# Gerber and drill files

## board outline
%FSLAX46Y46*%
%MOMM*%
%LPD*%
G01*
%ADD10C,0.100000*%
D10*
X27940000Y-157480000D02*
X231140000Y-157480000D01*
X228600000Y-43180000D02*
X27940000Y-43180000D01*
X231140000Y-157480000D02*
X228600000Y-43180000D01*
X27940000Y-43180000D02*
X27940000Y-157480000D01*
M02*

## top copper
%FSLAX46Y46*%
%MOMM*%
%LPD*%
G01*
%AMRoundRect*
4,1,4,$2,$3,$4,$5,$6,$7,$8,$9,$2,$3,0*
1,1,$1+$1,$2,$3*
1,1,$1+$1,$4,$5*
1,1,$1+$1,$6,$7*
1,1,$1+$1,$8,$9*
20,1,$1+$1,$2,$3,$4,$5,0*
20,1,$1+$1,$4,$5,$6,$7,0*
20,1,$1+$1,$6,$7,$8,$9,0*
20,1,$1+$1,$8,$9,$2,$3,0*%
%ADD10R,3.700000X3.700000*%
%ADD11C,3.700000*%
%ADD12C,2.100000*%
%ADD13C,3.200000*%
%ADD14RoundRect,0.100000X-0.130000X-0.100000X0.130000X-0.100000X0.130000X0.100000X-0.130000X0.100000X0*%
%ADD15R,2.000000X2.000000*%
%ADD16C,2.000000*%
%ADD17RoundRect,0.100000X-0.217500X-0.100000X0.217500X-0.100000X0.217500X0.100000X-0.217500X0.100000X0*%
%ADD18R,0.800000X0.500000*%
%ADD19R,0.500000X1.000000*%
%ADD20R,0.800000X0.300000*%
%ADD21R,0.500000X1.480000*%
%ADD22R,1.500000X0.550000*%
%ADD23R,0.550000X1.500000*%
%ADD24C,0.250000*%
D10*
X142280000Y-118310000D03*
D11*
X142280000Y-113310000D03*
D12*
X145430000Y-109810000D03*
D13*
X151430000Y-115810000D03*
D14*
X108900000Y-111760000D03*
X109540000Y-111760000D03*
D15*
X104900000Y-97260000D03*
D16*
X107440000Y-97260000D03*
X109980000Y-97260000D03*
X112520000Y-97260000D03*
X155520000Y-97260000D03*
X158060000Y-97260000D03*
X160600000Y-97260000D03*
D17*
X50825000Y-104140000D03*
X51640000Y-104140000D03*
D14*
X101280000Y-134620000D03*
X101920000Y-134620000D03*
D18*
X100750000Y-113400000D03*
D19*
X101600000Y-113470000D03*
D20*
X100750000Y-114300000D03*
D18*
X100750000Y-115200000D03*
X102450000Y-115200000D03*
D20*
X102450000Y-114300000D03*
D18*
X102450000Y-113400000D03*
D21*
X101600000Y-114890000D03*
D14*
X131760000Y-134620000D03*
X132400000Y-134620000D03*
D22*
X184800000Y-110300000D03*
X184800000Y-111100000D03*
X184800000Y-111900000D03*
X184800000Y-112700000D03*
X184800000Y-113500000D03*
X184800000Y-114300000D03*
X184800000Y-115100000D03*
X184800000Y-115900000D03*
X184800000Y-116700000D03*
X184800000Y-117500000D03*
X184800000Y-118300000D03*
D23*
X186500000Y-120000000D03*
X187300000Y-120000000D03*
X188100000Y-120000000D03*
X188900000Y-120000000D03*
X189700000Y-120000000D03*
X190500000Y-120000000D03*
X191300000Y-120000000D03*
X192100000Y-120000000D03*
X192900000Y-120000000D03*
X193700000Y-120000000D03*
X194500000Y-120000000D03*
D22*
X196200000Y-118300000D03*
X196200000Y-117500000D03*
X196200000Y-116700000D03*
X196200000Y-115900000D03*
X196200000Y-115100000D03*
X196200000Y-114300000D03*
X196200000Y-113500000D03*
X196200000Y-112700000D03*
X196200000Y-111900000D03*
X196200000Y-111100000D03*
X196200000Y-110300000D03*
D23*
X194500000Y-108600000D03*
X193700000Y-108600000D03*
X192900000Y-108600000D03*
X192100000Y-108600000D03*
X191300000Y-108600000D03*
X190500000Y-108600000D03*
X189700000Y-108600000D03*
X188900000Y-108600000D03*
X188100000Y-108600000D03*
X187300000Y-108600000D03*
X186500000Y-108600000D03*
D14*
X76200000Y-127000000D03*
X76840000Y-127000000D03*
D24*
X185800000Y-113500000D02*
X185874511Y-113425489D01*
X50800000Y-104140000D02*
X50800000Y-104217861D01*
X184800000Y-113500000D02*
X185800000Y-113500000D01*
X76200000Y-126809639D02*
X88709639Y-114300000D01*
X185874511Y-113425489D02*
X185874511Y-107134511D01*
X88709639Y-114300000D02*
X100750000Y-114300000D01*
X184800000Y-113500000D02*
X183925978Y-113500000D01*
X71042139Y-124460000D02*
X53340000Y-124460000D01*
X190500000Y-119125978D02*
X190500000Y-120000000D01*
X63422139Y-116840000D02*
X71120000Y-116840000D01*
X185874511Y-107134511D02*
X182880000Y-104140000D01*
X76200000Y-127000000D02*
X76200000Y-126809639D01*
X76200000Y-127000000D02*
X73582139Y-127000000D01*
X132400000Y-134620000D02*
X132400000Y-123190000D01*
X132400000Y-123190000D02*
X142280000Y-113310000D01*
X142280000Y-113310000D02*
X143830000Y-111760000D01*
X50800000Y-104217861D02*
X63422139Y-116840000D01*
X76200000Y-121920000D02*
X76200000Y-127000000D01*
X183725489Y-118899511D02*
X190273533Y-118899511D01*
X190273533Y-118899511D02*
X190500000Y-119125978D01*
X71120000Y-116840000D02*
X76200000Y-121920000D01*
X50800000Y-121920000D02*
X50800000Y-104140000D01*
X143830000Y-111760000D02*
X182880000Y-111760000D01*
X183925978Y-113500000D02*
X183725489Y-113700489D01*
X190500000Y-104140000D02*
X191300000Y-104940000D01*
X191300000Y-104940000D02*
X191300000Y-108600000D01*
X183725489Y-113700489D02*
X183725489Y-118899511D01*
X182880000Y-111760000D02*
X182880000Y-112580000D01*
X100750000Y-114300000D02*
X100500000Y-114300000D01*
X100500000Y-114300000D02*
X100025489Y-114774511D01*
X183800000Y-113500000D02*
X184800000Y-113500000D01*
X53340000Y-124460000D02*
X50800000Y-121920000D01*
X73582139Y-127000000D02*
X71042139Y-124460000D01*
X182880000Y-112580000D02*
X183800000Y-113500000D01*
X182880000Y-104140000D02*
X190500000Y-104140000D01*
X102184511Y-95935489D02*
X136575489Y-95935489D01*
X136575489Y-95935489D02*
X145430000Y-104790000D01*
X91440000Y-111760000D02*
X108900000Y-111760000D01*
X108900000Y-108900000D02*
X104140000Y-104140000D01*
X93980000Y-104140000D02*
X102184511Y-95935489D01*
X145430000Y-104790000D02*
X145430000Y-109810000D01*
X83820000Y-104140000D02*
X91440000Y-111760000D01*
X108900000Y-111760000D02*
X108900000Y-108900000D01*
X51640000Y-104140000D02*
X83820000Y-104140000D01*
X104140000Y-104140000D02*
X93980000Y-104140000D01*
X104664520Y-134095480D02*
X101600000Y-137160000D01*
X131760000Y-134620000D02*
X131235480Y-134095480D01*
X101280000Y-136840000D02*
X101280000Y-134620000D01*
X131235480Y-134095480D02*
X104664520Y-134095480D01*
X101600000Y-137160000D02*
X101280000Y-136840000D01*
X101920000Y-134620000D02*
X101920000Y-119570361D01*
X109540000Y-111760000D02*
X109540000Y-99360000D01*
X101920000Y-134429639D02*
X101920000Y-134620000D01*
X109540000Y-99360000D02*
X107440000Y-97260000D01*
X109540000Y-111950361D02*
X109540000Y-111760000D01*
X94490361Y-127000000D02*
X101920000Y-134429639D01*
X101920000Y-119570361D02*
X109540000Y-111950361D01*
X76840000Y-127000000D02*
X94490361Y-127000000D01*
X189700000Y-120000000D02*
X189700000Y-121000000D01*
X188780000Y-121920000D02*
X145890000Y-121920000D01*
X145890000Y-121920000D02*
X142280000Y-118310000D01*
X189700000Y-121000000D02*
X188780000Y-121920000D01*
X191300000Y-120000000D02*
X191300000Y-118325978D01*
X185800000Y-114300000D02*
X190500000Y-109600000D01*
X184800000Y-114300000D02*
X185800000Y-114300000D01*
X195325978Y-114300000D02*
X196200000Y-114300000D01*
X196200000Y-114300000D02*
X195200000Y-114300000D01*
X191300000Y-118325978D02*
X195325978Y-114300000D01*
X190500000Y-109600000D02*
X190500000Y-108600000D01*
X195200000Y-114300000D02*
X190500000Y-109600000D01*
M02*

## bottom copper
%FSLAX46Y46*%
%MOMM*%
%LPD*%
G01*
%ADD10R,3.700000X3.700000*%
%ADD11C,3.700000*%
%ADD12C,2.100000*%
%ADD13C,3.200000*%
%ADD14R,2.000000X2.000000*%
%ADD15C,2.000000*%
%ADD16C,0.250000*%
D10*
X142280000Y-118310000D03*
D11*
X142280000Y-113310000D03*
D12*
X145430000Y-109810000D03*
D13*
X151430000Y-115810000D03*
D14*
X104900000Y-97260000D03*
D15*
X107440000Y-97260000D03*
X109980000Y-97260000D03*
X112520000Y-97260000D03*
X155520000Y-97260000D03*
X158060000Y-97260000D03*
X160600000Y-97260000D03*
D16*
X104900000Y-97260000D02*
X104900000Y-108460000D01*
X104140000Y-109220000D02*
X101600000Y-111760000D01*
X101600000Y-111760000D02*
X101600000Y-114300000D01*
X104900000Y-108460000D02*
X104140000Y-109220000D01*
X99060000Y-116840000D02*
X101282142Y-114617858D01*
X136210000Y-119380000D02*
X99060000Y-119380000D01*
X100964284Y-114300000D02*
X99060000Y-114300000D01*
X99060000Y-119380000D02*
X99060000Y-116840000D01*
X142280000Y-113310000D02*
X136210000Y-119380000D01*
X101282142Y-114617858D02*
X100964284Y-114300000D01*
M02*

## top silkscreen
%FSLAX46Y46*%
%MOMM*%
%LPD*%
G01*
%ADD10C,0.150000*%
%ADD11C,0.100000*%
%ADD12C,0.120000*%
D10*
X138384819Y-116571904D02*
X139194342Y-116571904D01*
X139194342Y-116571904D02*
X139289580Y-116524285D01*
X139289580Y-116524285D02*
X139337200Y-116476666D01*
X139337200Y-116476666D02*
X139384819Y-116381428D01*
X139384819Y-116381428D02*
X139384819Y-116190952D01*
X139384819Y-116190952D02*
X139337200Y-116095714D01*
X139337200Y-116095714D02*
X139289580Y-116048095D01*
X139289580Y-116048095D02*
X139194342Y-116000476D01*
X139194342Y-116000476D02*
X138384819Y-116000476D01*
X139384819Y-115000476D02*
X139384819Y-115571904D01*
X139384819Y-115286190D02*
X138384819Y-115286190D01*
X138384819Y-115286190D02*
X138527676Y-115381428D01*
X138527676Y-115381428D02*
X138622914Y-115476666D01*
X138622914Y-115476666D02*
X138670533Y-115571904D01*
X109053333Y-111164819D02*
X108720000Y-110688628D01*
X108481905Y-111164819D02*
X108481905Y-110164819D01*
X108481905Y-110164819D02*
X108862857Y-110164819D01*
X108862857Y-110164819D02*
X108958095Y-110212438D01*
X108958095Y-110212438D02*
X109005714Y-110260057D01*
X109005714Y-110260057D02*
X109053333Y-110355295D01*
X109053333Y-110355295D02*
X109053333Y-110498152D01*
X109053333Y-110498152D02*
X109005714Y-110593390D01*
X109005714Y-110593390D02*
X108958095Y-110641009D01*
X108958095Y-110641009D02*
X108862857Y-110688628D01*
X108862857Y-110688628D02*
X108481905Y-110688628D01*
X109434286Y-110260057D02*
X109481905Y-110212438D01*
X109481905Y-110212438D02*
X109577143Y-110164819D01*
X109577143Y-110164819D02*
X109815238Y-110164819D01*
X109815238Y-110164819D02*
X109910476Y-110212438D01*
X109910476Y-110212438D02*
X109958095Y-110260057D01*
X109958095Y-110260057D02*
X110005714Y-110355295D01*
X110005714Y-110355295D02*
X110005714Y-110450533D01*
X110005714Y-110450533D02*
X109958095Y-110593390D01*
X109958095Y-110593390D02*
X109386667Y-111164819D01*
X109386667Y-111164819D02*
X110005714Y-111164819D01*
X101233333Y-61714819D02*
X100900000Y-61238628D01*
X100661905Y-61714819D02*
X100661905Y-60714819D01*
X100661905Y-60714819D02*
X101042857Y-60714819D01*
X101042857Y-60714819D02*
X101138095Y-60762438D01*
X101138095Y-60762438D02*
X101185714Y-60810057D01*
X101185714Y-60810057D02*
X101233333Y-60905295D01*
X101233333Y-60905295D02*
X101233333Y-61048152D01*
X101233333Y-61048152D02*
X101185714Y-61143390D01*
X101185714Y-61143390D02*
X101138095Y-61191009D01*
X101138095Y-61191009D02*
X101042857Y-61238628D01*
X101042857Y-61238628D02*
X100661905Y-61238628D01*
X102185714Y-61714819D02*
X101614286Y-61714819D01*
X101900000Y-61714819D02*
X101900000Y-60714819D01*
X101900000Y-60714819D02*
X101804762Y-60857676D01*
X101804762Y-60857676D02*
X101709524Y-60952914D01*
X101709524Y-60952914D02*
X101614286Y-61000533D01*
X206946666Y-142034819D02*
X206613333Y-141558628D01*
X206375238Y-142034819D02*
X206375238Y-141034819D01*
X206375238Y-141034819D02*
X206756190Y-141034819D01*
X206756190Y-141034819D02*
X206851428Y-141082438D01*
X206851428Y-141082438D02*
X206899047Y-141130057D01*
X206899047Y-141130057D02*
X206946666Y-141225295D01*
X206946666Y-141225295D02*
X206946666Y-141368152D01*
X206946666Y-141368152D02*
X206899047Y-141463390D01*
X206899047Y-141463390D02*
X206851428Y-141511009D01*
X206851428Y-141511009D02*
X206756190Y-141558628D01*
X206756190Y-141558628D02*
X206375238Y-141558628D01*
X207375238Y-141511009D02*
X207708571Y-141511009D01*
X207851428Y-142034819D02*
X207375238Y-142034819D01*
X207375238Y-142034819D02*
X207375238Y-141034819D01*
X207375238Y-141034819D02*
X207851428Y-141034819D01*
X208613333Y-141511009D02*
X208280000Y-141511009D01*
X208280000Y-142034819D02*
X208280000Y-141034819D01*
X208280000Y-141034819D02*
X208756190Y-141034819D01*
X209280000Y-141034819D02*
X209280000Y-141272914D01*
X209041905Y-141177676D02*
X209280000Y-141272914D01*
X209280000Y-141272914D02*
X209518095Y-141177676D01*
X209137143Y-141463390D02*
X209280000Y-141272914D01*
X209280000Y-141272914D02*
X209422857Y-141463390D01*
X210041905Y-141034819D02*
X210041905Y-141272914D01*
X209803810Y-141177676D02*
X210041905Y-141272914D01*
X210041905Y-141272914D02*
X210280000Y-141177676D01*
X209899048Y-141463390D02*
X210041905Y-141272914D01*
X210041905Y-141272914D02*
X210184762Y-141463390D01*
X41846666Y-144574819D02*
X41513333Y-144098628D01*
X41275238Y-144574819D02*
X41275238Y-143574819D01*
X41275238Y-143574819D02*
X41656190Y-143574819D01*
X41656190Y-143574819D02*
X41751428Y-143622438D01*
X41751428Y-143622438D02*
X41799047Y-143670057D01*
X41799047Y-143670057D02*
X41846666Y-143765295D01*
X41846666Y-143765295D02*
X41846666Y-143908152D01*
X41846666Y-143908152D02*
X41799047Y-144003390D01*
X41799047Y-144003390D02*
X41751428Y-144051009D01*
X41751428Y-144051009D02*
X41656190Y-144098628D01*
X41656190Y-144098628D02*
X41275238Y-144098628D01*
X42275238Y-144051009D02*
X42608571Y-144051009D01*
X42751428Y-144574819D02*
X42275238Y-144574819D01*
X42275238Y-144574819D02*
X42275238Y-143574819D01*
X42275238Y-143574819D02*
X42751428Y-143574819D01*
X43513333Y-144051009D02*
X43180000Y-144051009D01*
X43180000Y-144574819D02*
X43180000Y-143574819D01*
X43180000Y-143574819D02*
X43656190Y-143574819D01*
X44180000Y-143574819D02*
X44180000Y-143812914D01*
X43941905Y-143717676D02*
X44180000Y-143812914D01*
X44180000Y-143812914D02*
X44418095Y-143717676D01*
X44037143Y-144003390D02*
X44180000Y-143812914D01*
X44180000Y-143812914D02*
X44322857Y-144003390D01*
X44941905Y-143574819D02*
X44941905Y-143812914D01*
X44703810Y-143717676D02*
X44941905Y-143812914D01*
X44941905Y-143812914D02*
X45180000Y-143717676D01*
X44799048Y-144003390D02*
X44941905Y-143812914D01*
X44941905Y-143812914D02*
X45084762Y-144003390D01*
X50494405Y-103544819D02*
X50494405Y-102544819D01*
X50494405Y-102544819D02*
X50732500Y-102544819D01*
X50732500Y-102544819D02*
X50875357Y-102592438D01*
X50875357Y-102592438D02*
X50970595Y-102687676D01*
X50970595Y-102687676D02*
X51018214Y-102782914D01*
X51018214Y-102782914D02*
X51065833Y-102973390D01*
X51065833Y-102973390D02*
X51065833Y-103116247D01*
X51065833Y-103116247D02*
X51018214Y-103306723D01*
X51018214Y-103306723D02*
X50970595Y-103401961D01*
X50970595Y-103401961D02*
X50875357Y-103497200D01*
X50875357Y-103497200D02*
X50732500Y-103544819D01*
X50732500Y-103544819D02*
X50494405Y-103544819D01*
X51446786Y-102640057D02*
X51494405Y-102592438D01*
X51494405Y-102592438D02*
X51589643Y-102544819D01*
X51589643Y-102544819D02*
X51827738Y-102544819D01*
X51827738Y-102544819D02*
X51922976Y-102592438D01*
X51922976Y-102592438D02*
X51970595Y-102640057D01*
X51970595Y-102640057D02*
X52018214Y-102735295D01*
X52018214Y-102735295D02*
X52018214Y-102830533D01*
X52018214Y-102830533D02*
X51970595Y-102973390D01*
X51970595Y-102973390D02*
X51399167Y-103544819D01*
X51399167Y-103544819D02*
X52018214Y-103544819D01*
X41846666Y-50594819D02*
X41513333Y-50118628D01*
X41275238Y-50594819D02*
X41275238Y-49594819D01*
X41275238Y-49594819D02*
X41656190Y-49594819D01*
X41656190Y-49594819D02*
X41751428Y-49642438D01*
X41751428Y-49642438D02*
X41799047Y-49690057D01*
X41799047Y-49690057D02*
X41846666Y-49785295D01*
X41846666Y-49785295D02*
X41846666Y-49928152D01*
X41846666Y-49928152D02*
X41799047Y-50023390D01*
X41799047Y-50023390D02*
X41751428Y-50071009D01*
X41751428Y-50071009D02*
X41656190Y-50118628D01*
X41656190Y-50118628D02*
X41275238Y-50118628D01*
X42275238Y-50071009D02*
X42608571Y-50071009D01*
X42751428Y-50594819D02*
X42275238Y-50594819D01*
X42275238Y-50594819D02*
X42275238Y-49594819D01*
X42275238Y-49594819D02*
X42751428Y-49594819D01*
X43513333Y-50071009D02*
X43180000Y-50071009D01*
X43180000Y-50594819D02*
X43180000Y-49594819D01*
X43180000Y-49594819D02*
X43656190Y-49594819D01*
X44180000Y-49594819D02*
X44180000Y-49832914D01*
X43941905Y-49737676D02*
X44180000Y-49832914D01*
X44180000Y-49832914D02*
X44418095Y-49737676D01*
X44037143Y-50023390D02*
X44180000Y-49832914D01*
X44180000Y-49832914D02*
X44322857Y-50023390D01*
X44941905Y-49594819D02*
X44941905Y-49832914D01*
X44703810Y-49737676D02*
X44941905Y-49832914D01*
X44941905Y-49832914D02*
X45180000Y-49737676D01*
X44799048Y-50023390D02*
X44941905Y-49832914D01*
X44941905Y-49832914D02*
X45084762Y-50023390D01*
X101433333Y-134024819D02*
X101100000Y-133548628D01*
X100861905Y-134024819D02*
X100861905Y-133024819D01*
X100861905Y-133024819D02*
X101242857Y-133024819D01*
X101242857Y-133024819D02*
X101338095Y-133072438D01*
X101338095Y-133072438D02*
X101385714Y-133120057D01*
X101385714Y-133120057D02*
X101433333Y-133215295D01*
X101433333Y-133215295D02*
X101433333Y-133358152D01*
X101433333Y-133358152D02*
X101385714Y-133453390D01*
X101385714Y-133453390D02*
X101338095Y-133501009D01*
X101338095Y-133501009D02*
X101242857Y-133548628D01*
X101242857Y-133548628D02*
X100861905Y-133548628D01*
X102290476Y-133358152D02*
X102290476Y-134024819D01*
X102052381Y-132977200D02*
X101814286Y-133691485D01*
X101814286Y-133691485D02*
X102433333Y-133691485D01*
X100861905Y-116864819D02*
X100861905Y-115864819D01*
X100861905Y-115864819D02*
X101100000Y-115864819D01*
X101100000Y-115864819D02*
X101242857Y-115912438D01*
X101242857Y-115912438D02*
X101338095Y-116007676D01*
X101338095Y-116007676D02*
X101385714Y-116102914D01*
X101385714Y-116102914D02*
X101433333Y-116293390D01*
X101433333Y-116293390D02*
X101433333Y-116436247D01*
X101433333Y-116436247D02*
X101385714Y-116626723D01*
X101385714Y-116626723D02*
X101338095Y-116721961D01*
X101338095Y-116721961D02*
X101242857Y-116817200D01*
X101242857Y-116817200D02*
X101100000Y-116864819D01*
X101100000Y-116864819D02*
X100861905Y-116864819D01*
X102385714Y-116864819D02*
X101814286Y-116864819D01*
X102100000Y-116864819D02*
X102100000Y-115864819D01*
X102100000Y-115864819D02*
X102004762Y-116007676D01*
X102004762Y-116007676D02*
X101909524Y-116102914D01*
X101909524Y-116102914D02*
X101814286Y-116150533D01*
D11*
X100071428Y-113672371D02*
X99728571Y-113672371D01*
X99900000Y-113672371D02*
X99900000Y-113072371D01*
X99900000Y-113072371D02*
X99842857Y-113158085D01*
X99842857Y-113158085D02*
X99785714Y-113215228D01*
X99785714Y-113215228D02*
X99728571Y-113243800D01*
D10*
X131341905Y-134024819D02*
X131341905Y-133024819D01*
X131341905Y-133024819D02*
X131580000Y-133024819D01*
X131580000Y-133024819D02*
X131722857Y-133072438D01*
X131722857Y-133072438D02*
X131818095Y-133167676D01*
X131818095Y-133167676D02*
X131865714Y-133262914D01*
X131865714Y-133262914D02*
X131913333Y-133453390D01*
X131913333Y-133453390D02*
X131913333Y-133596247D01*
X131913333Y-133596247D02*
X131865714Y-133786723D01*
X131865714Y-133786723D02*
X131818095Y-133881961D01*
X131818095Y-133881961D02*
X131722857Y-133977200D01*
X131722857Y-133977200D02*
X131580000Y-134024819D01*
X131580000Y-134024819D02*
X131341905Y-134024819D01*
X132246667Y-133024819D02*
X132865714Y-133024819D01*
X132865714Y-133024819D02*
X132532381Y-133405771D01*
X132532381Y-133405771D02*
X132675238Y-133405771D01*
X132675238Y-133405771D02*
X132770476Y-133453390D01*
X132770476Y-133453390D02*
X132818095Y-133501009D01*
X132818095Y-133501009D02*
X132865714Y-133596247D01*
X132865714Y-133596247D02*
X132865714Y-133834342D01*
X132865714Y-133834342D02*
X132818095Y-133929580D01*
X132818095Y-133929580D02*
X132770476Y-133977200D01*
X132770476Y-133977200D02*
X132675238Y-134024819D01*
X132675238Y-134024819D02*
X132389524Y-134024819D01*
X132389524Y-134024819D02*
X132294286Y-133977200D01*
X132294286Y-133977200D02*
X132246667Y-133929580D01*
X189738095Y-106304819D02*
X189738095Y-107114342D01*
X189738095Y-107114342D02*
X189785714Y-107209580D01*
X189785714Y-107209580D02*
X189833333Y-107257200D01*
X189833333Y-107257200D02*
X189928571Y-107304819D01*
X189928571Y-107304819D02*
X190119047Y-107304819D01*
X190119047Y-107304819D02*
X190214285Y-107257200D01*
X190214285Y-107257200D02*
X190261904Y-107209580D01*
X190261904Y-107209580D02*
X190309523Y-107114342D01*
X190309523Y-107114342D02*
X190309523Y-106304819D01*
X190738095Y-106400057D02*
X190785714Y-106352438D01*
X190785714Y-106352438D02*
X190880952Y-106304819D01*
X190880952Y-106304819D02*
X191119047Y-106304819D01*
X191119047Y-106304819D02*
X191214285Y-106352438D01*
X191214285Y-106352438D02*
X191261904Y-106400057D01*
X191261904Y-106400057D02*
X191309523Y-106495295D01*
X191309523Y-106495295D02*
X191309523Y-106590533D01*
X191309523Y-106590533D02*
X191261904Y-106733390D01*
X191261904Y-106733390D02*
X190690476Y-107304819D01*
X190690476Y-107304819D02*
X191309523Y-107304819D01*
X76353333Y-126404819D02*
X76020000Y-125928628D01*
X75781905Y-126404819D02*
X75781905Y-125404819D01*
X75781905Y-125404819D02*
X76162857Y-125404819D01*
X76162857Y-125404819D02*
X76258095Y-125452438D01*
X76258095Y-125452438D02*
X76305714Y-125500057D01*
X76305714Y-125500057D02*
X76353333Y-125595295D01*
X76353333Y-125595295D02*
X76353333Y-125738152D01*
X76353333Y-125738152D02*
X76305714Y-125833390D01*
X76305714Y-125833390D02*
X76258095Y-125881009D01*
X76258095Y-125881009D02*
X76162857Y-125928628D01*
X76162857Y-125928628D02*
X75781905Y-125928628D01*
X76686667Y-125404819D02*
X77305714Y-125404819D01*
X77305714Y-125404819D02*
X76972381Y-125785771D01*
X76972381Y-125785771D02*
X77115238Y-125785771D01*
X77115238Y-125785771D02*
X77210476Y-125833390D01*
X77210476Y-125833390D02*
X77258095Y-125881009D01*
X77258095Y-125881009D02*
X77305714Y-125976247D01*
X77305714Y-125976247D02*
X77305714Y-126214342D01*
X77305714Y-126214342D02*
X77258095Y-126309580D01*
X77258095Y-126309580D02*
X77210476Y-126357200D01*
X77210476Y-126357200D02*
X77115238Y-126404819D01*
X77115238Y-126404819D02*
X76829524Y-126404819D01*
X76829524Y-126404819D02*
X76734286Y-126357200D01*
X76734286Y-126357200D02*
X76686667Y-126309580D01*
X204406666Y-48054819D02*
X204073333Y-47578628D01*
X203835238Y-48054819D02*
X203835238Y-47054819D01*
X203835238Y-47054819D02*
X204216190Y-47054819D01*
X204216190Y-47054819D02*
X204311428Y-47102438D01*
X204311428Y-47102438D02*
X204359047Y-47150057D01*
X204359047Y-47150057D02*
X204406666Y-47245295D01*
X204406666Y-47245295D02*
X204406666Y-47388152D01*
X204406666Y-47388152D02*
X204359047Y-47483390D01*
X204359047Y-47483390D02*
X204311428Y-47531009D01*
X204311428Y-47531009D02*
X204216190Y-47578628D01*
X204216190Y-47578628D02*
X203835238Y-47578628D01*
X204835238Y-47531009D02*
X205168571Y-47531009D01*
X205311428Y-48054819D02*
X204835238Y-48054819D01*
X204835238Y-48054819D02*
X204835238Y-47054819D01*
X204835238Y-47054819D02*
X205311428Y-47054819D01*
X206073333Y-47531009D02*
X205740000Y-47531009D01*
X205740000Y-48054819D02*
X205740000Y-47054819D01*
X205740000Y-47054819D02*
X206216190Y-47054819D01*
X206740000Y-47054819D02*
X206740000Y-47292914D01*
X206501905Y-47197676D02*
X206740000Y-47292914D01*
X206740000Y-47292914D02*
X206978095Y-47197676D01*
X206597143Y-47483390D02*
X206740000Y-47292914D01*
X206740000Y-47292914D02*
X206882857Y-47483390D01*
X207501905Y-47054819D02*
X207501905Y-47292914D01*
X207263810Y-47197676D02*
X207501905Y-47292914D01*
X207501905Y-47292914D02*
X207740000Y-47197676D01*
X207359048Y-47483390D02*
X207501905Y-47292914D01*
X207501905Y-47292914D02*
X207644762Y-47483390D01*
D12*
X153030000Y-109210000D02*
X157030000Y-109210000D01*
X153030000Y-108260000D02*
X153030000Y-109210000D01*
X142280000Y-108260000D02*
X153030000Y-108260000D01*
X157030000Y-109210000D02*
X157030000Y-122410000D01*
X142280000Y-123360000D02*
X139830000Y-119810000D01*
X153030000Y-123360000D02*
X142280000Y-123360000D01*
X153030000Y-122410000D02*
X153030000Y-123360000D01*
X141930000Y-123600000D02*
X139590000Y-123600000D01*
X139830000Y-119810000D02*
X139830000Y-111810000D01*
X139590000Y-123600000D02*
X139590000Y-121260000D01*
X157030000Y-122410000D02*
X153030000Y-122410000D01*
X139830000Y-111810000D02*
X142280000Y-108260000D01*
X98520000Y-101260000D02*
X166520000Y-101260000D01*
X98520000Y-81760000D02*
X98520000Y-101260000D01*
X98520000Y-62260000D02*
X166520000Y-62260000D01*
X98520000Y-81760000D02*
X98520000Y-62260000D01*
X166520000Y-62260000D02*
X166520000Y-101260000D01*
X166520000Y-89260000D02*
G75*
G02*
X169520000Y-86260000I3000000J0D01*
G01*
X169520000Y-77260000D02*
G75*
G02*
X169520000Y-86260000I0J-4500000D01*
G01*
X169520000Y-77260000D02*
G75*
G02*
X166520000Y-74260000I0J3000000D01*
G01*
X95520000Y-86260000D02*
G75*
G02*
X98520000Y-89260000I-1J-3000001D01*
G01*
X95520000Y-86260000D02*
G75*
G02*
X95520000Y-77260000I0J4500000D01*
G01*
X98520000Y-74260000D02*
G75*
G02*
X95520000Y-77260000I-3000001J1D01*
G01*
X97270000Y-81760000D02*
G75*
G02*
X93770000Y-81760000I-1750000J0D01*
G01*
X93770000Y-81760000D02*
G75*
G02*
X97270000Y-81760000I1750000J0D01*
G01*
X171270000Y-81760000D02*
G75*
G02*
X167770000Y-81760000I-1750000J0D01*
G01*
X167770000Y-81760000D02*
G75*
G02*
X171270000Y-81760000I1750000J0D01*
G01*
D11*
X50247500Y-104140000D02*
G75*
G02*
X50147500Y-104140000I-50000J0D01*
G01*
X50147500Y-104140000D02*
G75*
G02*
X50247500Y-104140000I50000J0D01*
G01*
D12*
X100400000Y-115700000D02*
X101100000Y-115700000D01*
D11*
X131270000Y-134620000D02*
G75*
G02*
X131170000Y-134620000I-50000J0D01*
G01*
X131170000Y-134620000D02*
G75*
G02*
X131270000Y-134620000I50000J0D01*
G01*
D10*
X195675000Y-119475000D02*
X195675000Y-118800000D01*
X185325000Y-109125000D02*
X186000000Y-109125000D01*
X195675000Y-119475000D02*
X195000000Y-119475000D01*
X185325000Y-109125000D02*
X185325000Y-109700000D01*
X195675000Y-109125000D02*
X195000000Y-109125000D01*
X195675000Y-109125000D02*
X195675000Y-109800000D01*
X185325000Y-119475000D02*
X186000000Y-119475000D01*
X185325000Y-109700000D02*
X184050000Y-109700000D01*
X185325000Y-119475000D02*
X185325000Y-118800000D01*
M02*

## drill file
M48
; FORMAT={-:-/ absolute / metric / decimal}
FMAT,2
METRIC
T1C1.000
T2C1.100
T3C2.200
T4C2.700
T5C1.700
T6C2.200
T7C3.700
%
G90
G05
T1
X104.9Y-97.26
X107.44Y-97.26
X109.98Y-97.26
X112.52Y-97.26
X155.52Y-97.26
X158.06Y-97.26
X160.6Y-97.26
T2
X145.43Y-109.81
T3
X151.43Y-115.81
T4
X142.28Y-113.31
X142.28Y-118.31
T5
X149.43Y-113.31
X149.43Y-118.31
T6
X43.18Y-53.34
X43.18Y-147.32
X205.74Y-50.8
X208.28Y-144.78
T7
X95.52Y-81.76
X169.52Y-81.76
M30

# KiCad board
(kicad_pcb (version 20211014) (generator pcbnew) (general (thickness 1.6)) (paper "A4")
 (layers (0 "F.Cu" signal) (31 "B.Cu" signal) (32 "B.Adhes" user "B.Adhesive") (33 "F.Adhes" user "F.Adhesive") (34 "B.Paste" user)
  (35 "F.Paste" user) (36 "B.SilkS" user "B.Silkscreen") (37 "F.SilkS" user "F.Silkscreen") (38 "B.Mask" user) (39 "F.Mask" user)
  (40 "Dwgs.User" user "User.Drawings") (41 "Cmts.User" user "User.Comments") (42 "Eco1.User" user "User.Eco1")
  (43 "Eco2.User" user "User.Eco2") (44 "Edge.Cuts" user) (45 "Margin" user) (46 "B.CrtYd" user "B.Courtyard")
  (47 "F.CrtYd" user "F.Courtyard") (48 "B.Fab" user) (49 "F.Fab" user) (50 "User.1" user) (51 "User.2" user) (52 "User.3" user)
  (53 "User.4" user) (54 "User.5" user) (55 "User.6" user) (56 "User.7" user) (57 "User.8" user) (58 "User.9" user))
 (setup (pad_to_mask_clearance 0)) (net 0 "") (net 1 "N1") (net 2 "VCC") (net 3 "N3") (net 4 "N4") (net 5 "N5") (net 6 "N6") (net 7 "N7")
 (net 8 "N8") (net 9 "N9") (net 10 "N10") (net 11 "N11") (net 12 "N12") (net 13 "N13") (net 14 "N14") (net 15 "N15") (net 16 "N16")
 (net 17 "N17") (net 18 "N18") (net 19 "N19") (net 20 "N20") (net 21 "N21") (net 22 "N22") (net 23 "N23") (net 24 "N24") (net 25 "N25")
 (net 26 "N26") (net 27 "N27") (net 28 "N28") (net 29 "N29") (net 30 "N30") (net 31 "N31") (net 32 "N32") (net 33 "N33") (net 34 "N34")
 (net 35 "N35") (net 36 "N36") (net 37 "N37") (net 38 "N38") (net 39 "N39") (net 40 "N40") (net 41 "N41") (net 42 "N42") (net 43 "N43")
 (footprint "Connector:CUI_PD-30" (layer "F.Cu") (at 142.28 118.31 90)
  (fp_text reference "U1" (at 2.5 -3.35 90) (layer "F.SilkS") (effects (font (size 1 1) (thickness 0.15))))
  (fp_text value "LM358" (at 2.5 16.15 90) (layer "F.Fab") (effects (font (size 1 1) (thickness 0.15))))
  (fp_line (start 9.1 10.75) (end 9.1 14.75) (layer "F.SilkS") (width 0.12))
  (fp_line (start 10.05 10.75) (end 9.1 10.75) (layer "F.SilkS") (width 0.12))
  (fp_line (start 10.05 0) (end 10.05 10.75) (layer "F.SilkS") (width 0.12))
  (fp_line (start 9.1 14.75) (end -4.1 14.75) (layer "F.SilkS") (width 0.12))
  (fp_line (start -5.05 0) (end -1.5 -2.45) (layer "F.SilkS") (width 0.12))
  (fp_line (start -5.05 10.75) (end -5.05 0) (layer "F.SilkS") (width 0.12))
  (fp_line (start -4.1 10.75) (end -5.05 10.75) (layer "F.SilkS") (width 0.12))
  (fp_line (start -5.29 -0.35) (end -5.29 -2.69) (layer "F.SilkS") (width 0.12))
  (fp_line (start -1.5 -2.45) (end 6.5 -2.45) (layer "F.SilkS") (width 0.12))
  (fp_line (start -5.29 -2.69) (end -2.95 -2.69) (layer "F.SilkS") (width 0.12))
  (fp_line (start -4.1 14.75) (end -4.1 10.75) (layer "F.SilkS") (width 0.12))
  (fp_line (start 6.5 -2.45) (end 10.05 0) (layer "F.SilkS") (width 0.12))
  (pad "" np_thru_hole circle (at 5 7.15 270) (size 1.7 1.7) (drill 1.7) (layers *.Cu *.Mask))
  (pad "" np_thru_hole circle (at 0 7.15 270) (size 1.7 1.7) (drill 1.7) (layers *.Cu *.Mask))
  (pad "1" thru_hole rect (at 0 0 270) (size 3.7 3.7) (drill 2.7) (layers *.Cu *.Mask) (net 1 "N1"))
  (pad "2" thru_hole circle (at 5 0 270) (size 3.7 3.7) (drill 2.7) (layers *.Cu *.Mask) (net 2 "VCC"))
  (pad "3" thru_hole circle (at 8.5 3.15 270) (size 2.1 2.1) (drill 1.1) (layers *.Cu *.Mask) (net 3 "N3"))
  (pad "4" thru_hole circle (at 2.5 9.15 270) (size 3.2 3.2) (drill 2.2) (layers *.Cu *.Mask)))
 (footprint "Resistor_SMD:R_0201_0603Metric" (layer "F.Cu") (at 109.22 111.76)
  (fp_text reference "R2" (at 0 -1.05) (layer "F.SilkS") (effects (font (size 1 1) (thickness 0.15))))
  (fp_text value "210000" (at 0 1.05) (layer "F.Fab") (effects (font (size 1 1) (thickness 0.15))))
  (pad "" smd roundrect (at 0.345 0) (size 0.318 0.36) (layers "F.Paste") (roundrect_rratio 0.25))
  (pad "" smd roundrect (at -0.345 0) (size 0.318 0.36) (layers "F.Paste") (roundrect_rratio 0.25))
  (pad "1" smd roundrect (at -0.32 0) (size 0.46 0.4) (layers "F.Cu" "F.Mask") (roundrect_rratio 0.25) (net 3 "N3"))
  (pad "2" smd roundrect (at 0.32 0) (size 0.46 0.4) (layers "F.Cu" "F.Mask") (roundrect_rratio 0.25) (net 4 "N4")))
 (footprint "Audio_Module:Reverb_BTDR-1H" (layer "F.Cu") (at 104.9 97.26)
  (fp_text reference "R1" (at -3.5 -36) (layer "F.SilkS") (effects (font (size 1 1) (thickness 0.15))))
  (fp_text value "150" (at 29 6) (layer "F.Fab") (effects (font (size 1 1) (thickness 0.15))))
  (fp_line (start -6.38 4) (end 61.62 4) (layer "F.SilkS") (width 0.12))
  (fp_line (start -6.38 -15.5) (end -6.38 4) (layer "F.SilkS") (width 0.12))
  (fp_line (start -6.38 -35) (end 61.62 -35) (layer "F.SilkS") (width 0.12))
  (fp_line (start -6.38 -15.5) (end -6.38 -35) (layer "F.SilkS") (width 0.12))
  (fp_line (start 61.62 -35) (end 61.62 4) (layer "F.SilkS") (width 0.12))
  (fp_arc (start 61.62 -8) (mid 62.49868 -10.12132) (end 64.62 -11) (layer "F.SilkS") (width 0.12))
  (fp_arc (start 64.62 -20) (mid 69.12 -15.5) (end 64.62 -11) (layer "F.SilkS") (width 0.12))
  (fp_arc (start 64.62 -20) (mid 62.49868 -20.87868) (end 61.62 -23) (layer "F.SilkS") (width 0.12))
  (fp_arc (start -9.38 -11) (mid -7.25868 -10.12132) (end -6.38 -8) (layer "F.SilkS") (width 0.12))
  (fp_arc (start -9.38 -11) (mid -13.88 -15.5) (end -9.38 -20) (layer "F.SilkS") (width 0.12))
  (fp_arc (start -6.38 -23) (mid -7.25868 -20.87868) (end -9.38 -20) (layer "F.SilkS") (width 0.12))
  (fp_circle (center -9.38 -15.5) (end -7.63 -15.5) (layer "F.SilkS") (width 0.12) (fill none))
  (fp_circle (center 64.62 -15.5) (end 66.37 -15.5) (layer "F.SilkS") (width 0.12) (fill none))
  (pad "" np_thru_hole circle (at 64.62 -15.5) (size 3.7 3.7) (drill 3.7) (layers *.Cu *.Mask))
  (pad "" np_thru_hole circle (at -9.38 -15.5) (size 3.7 3.7) (drill 3.7) (layers *.Cu *.Mask))
  (pad "1" thru_hole rect (at 0 0) (size 2 2) (drill 1) (layers *.Cu *.Mask) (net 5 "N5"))
  (pad "2" thru_hole circle (at 2.54 0) (size 2 2) (drill 1) (layers *.Cu *.Mask) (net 4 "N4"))
  (pad "3" thru_hole circle (at 5.08 0) (size 2 2) (drill 1) (layers *.Cu *.Mask))
  (pad "4" thru_hole circle (at 7.62 0) (size 2 2) (drill 1) (layers *.Cu *.Mask))
  (pad "5" thru_hole circle (at 50.62 0) (size 2 2) (drill 1) (layers *.Cu *.Mask))
  (pad "6" thru_hole circle (at 53.16 0) (size 2 2) (drill 1) (layers *.Cu *.Mask))
  (pad "7" thru_hole circle (at 55.7 0) (size 2 2) (drill 1) (layers *.Cu *.Mask)))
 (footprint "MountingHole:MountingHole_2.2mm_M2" (layer "F.Cu") (at 208.28 144.78)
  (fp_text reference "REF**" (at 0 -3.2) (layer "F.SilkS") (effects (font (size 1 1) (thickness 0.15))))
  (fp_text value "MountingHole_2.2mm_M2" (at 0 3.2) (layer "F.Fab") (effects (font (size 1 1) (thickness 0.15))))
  (pad "" np_thru_hole circle (at 0 0) (size 2.2 2.2) (drill 2.2) (layers *.Cu *.Mask)))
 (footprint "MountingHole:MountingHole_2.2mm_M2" (layer "F.Cu") (at 43.18 147.32)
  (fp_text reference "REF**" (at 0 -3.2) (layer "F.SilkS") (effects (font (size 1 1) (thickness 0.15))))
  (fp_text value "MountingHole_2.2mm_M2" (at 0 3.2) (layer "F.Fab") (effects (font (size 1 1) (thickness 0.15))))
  (pad "" np_thru_hole circle (at 0 0) (size 2.2 2.2) (drill 2.2) (layers *.Cu *.Mask)))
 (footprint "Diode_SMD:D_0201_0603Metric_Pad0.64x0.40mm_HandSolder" (layer "F.Cu") (at 51.2325 104.14)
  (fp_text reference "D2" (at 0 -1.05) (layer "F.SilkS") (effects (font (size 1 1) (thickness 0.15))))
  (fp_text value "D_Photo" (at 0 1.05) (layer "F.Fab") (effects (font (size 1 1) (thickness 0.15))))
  (fp_circle (center -1.035 0) (end -0.985 0) (layer "F.SilkS") (width 0.1) (fill none))
  (pad "" smd roundrect (at -0.4325 0) (size 0.458 0.36) (layers "F.Paste") (roundrect_rratio 0.25))
  (pad "" smd roundrect (at 0.4325 0) (size 0.458 0.36) (layers "F.Paste") (roundrect_rratio 0.25))
  (pad "1" smd roundrect (at -0.4075 0) (size 0.635 0.4) (layers "F.Cu" "F.Mask") (roundrect_rratio 0.25) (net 2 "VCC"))
  (pad "2" smd roundrect (at 0.4075 0) (size 0.635 0.4) (layers "F.Cu" "F.Mask") (roundrect_rratio 0.25) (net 3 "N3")))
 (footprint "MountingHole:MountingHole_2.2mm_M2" (layer "F.Cu") (at 43.18 53.34)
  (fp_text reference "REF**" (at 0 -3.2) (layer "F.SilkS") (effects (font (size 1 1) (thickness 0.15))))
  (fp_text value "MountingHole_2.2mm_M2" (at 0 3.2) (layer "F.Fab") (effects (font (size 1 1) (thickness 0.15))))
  (pad "" np_thru_hole circle (at 0 0) (size 2.2 2.2) (drill 2.2) (layers *.Cu *.Mask)))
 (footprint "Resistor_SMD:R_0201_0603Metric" (layer "F.Cu") (at 101.6 134.62)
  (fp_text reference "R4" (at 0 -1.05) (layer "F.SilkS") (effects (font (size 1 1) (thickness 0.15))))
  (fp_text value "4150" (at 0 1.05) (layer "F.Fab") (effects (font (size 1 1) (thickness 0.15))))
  (pad "" smd roundrect (at -0.345 0) (size 0.318 0.36) (layers "F.Paste") (roundrect_rratio 0.25))
  (pad "" smd roundrect (at 0.345 0) (size 0.318 0.36) (layers "F.Paste") (roundrect_rratio 0.25))
  (pad "1" smd roundrect (at -0.32 0) (size 0.46 0.4) (layers "F.Cu" "F.Mask") (roundrect_rratio 0.25) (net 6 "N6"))
  (pad "2" smd roundrect (at 0.32 0) (size 0.46 0.4) (layers "F.Cu" "F.Mask") (roundrect_rratio 0.25) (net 4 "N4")))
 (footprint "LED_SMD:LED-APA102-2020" (layer "F.Cu") (at 101.6 114.3)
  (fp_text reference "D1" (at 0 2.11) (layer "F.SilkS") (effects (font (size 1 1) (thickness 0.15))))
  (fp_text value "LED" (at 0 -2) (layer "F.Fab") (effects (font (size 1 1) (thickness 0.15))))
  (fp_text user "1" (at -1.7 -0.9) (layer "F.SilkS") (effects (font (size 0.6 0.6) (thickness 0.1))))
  (fp_line (start -1.2 1.4) (end -0.5 1.4) (layer "F.SilkS") (width 0.12))
  (pad "1" smd rect (at -0.85 -0.9) (size 0.8 0.5) (layers "F.Cu" "F.Paste" "F.Mask") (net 5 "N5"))
  (pad "1" smd rect (at 0 -0.83 90) (size 1 0.5) (layers "F.Cu" "F.Paste" "F.Mask") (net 5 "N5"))
  (pad "2" smd rect (at -0.85 0) (size 0.8 0.3) (layers "F.Cu" "F.Paste" "F.Mask") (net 2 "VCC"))
  (pad "3" smd rect (at -0.85 0.9) (size 0.8 0.5) (layers "F.Cu" "F.Paste" "F.Mask"))
  (pad "4" smd rect (at 0.85 0.9) (size 0.8 0.5) (layers "F.Cu" "F.Paste" "F.Mask"))
  (pad "5" smd rect (at 0.85 0) (size 0.8 0.3) (layers "F.Cu" "F.Paste" "F.Mask"))
  (pad "6" smd rect (at 0.85 -0.9) (size 0.8 0.5) (layers "F.Cu" "F.Paste" "F.Mask"))
  (pad "6" smd rect (at 0 0.59 90) (size 1.48 0.5) (layers "F.Cu" "F.Paste" "F.Mask")))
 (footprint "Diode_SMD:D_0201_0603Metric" (layer "F.Cu") (at 132.08 134.62)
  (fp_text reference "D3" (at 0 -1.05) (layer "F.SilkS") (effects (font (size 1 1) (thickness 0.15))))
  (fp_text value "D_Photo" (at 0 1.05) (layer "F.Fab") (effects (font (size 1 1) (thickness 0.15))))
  (fp_circle (center -0.86 0) (end -0.81 0) (layer "F.SilkS") (width 0.1) (fill none))
  (pad "" smd roundrect (at 0.345 0) (size 0.318 0.36) (layers "F.Paste") (roundrect_rratio 0.25))
  (pad "" smd roundrect (at -0.345 0) (size 0.318 0.36) (layers "F.Paste") (roundrect_rratio 0.25))
  (pad "1" smd roundrect (at -0.32 0) (size 0.46 0.4) (layers "F.Cu" "F.Mask") (roundrect_rratio 0.25) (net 6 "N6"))
  (pad "2" smd roundrect (at 0.32 0) (size 0.46 0.4) (layers "F.Cu" "F.Mask") (roundrect_rratio 0.25) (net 2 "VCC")))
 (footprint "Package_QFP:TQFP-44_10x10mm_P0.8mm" (layer "F.Cu") (at 190.5 114.3)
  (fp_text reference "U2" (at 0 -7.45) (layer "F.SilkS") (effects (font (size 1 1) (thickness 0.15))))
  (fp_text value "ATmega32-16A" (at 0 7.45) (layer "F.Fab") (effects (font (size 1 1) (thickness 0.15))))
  (fp_line (start 5.175 5.175) (end 5.175 4.5) (layer "F.SilkS") (width 0.15))
  (fp_line (start -5.175 -5.175) (end -4.5 -5.175) (layer "F.SilkS") (width 0.15))
  (fp_line (start 5.175 5.175) (end 4.5 5.175) (layer "F.SilkS") (width 0.15))
  (fp_line (start -5.175 -5.175) (end -5.175 -4.6) (layer "F.SilkS") (width 0.15))
  (fp_line (start 5.175 -5.175) (end 4.5 -5.175) (layer "F.SilkS") (width 0.15))
  (fp_line (start 5.175 -5.175) (end 5.175 -4.5) (layer "F.SilkS") (width 0.15))
  (fp_line (start -5.175 5.175) (end -4.5 5.175) (layer "F.SilkS") (width 0.15))
  (fp_line (start -5.175 -4.6) (end -6.45 -4.6) (layer "F.SilkS") (width 0.15))
  (fp_line (start -5.175 5.175) (end -5.175 4.5) (layer "F.SilkS") (width 0.15))
  (pad "1" smd rect (at -5.7 -4) (size 1.5 0.55) (layers "F.Cu" "F.Paste" "F.Mask") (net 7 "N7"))
  (pad "2" smd rect (at -5.7 -3.2) (size 1.5 0.55) (layers "F.Cu" "F.Paste" "F.Mask") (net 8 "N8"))
  (pad "3" smd rect (at -5.7 -2.4) (size 1.5 0.55) (layers "F.Cu" "F.Paste" "F.Mask") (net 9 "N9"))
  (pad "4" smd rect (at -5.7 -1.6) (size 1.5 0.55) (layers "F.Cu" "F.Paste" "F.Mask") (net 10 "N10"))
  (pad "5" smd rect (at -5.7 -0.8) (size 1.5 0.55) (layers "F.Cu" "F.Paste" "F.Mask") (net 2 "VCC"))
  (pad "6" smd rect (at -5.7 0) (size 1.5 0.55) (layers "F.Cu" "F.Paste" "F.Mask") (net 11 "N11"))
  (pad "7" smd rect (at -5.7 0.8) (size 1.5 0.55) (layers "F.Cu" "F.Paste" "F.Mask") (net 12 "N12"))
  (pad "8" smd rect (at -5.7 1.6) (size 1.5 0.55) (layers "F.Cu" "F.Paste" "F.Mask") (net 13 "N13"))
  (pad "9" smd rect (at -5.7 2.4) (size 1.5 0.55) (layers "F.Cu" "F.Paste" "F.Mask") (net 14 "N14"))
  (pad "10" smd rect (at -5.7 3.2) (size 1.5 0.55) (layers "F.Cu" "F.Paste" "F.Mask") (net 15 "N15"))
  (pad "11" smd rect (at -5.7 4) (size 1.5 0.55) (layers "F.Cu" "F.Paste" "F.Mask") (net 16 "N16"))
  (pad "12" smd rect (at -4 5.7 90) (size 1.5 0.55) (layers "F.Cu" "F.Paste" "F.Mask") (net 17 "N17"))
  (pad "13" smd rect (at -3.2 5.7 90) (size 1.5 0.55) (layers "F.Cu" "F.Paste" "F.Mask") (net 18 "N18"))
  (pad "14" smd rect (at -2.4 5.7 90) (size 1.5 0.55) (layers "F.Cu" "F.Paste" "F.Mask") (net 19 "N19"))
  (pad "15" smd rect (at -1.6 5.7 90) (size 1.5 0.55) (layers "F.Cu" "F.Paste" "F.Mask") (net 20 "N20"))
  (pad "16" smd rect (at -0.8 5.7 90) (size 1.5 0.55) (layers "F.Cu" "F.Paste" "F.Mask") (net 1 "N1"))
  (pad "17" smd rect (at 0 5.7 90) (size 1.5 0.55) (layers "F.Cu" "F.Paste" "F.Mask") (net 2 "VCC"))
  (pad "18" smd rect (at 0.8 5.7 90) (size 1.5 0.55) (layers "F.Cu" "F.Paste" "F.Mask") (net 11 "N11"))
  (pad "19" smd rect (at 1.6 5.7 90) (size 1.5 0.55) (layers "F.Cu" "F.Paste" "F.Mask") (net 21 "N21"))
  (pad "20" smd rect (at 2.4 5.7 90) (size 1.5 0.55) (layers "F.Cu" "F.Paste" "F.Mask") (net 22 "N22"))
  (pad "21" smd rect (at 3.2 5.7 90) (size 1.5 0.55) (layers "F.Cu" "F.Paste" "F.Mask") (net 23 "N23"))
  (pad "22" smd rect (at 4 5.7 90) (size 1.5 0.55) (layers "F.Cu" "F.Paste" "F.Mask") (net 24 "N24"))
  (pad "23" smd rect (at 5.7 4) (size 1.5 0.55) (layers "F.Cu" "F.Paste" "F.Mask") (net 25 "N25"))
  (pad "24" smd rect (at 5.7 3.2) (size 1.5 0.55) (layers "F.Cu" "F.Paste" "F.Mask") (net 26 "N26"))
  (pad "25" smd rect (at 5.7 2.4) (size 1.5 0.55) (layers "F.Cu" "F.Paste" "F.Mask") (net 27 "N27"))
  (pad "26" smd rect (at 5.7 1.6) (size 1.5 0.55) (layers "F.Cu" "F.Paste" "F.Mask") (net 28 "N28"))
  (pad "27" smd rect (at 5.7 0.8) (size 1.5 0.55) (layers "F.Cu" "F.Paste" "F.Mask") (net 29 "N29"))
  (pad "28" smd rect (at 5.7 0) (size 1.5 0.55) (layers "F.Cu" "F.Paste" "F.Mask") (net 11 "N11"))
  (pad "29" smd rect (at 5.7 -0.8) (size 1.5 0.55) (layers "F.Cu" "F.Paste" "F.Mask") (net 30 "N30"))
  (pad "30" smd rect (at 5.7 -1.6) (size 1.5 0.55) (layers "F.Cu" "F.Paste" "F.Mask") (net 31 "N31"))
  (pad "31" smd rect (at 5.7 -2.4) (size 1.5 0.55) (layers "F.Cu" "F.Paste" "F.Mask") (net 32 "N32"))
  (pad "32" smd rect (at 5.7 -3.2) (size 1.5 0.55) (layers "F.Cu" "F.Paste" "F.Mask") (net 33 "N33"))
  (pad "33" smd rect (at 5.7 -4) (size 1.5 0.55) (layers "F.Cu" "F.Paste" "F.Mask") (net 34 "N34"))
  (pad "34" smd rect (at 4 -5.7 90) (size 1.5 0.55) (layers "F.Cu" "F.Paste" "F.Mask") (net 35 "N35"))
  (pad "35" smd rect (at 3.2 -5.7 90) (size 1.5 0.55) (layers "F.Cu" "F.Paste" "F.Mask") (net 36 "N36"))
  (pad "36" smd rect (at 2.4 -5.7 90) (size 1.5 0.55) (layers "F.Cu" "F.Paste" "F.Mask") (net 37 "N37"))
  (pad "37" smd rect (at 1.6 -5.7 90) (size 1.5 0.55) (layers "F.Cu" "F.Paste" "F.Mask") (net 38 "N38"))
  (pad "38" smd rect (at 0.8 -5.7 90) (size 1.5 0.55) (layers "F.Cu" "F.Paste" "F.Mask") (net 2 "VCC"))
  (pad "39" smd rect (at 0 -5.7 90) (size 1.5 0.55) (layers "F.Cu" "F.Paste" "F.Mask") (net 11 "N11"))
  (pad "40" smd rect (at -0.8 -5.7 90) (size 1.5 0.55) (layers "F.Cu" "F.Paste" "F.Mask") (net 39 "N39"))
  (pad "41" smd rect (at -1.6 -5.7 90) (size 1.5 0.55) (layers "F.Cu" "F.Paste" "F.Mask") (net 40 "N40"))
  (pad "42" smd rect (at -2.4 -5.7 90) (size 1.5 0.55) (layers "F.Cu" "F.Paste" "F.Mask") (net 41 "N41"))
  (pad "43" smd rect (at -3.2 -5.7 90) (size 1.5 0.55) (layers "F.Cu" "F.Paste" "F.Mask") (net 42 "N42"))
  (pad "44" smd rect (at -4 -5.7 90) (size 1.5 0.55) (layers "F.Cu" "F.Paste" "F.Mask") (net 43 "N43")))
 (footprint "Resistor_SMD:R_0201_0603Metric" (layer "F.Cu") (at 76.52 127)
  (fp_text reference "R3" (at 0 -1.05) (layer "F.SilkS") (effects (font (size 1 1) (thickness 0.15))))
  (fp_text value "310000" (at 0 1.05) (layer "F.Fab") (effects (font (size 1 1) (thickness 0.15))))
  (pad "" smd roundrect (at -0.345 0) (size 0.318 0.36) (layers "F.Paste") (roundrect_rratio 0.25))
  (pad "" smd roundrect (at 0.345 0) (size 0.318 0.36) (layers "F.Paste") (roundrect_rratio 0.25))
  (pad "1" smd roundrect (at -0.32 0) (size 0.46 0.4) (layers "F.Cu" "F.Mask") (roundrect_rratio 0.25) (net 2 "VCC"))
  (pad "2" smd roundrect (at 0.32 0) (size 0.46 0.4) (layers "F.Cu" "F.Mask") (roundrect_rratio 0.25) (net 4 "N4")))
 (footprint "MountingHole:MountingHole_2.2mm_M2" (layer "F.Cu") (at 205.74 50.8)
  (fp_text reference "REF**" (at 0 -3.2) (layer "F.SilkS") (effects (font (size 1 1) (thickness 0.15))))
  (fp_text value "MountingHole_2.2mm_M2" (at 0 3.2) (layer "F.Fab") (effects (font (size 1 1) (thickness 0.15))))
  (pad "" np_thru_hole circle (at 0 0) (size 2.2 2.2) (drill 2.2) (layers *.Cu *.Mask)))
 (gr_line (start 27.94 157.48) (end 231.14 157.48) (layer "Edge.Cuts") (width 0.1))
 (gr_line (start 228.6 43.18) (end 27.94 43.18) (layer "Edge.Cuts") (width 0.1))
 (gr_line (start 231.14 157.48) (end 228.6 43.18) (layer "Edge.Cuts") (width 0.1))
 (gr_line (start 27.94 43.18) (end 27.94 157.48) (layer "Edge.Cuts") (width 0.1))
 (segment (start 104.9 97.26) (end 104.9 108.46) (width 0.25) (layer "B.Cu") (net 5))
 (segment (start 104.14 109.22) (end 101.6 111.76) (width 0.25) (layer "B.Cu") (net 5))
 (segment (start 101.6 111.76) (end 101.6 114.3) (width 0.25) (layer "B.Cu") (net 5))
 (segment (start 104.9 108.46) (end 104.14 109.22) (width 0.25) (layer "B.Cu") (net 5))
 (segment (start 185.8 113.5) (end 185.874511 113.425489) (width 0.25) (layer "F.Cu") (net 2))
 (segment (start 50.8 104.14) (end 50.8 104.217861) (width 0.25) (layer "F.Cu") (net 2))
 (segment (start 184.8 113.5) (end 185.8 113.5) (width 0.25) (layer "F.Cu") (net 2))
 (segment (start 76.2 126.809639) (end 88.709639 114.3) (width 0.25) (layer "F.Cu") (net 2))
 (segment (start 185.874511 113.425489) (end 185.874511 107.134511) (width 0.25) (layer "F.Cu") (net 2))
 (segment (start 88.709639 114.3) (end 100.75 114.3) (width 0.25) (layer "F.Cu") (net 2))
 (segment (start 184.8 113.5) (end 183.925978 113.5) (width 0.25) (layer "F.Cu") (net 2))
 (segment (start 71.042139 124.46) (end 53.34 124.46) (width 0.25) (layer "F.Cu") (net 2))
 (segment (start 190.5 119.125978) (end 190.5 120) (width 0.25) (layer "F.Cu") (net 2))
 (segment (start 63.422139 116.84) (end 71.12 116.84) (width 0.25) (layer "F.Cu") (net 2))
 (segment (start 185.874511 107.134511) (end 182.88 104.14) (width 0.25) (layer "F.Cu") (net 2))
 (segment (start 76.2 127) (end 76.2 126.809639) (width 0.25) (layer "F.Cu") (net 2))
 (segment (start 76.2 127) (end 73.582139 127) (width 0.25) (layer "F.Cu") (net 2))
 (segment (start 132.4 134.62) (end 132.4 123.19) (width 0.25) (layer "F.Cu") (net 2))
 (segment (start 132.4 123.19) (end 142.28 113.31) (width 0.25) (layer "F.Cu") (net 2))
 (segment (start 142.28 113.31) (end 143.83 111.76) (width 0.25) (layer "F.Cu") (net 2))
 (segment (start 50.8 104.217861) (end 63.422139 116.84) (width 0.25) (layer "F.Cu") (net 2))
 (segment (start 76.2 121.92) (end 76.2 127) (width 0.25) (layer "F.Cu") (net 2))
 (segment (start 183.725489 118.899511) (end 190.273533 118.899511) (width 0.25) (layer "F.Cu") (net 2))
 (segment (start 190.273533 118.899511) (end 190.5 119.125978) (width 0.25) (layer "F.Cu") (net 2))
 (segment (start 71.12 116.84) (end 76.2 121.92) (width 0.25) (layer "F.Cu") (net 2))
 (segment (start 50.8 121.92) (end 50.8 104.14) (width 0.25) (layer "F.Cu") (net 2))
 (segment (start 143.83 111.76) (end 182.88 111.76) (width 0.25) (layer "F.Cu") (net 2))
 (segment (start 183.925978 113.5) (end 183.725489 113.700489) (width 0.25) (layer "F.Cu") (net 2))
 (segment (start 190.5 104.14) (end 191.3 104.94) (width 0.25) (layer "F.Cu") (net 2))
 (segment (start 191.3 104.94) (end 191.3 108.6) (width 0.25) (layer "F.Cu") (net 2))
 (segment (start 183.725489 113.700489) (end 183.725489 118.899511) (width 0.25) (layer "F.Cu") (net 2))
 (segment (start 182.88 111.76) (end 182.88 112.58) (width 0.25) (layer "F.Cu") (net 2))
 (segment (start 100.75 114.3) (end 100.5 114.3) (width 0.25) (layer "F.Cu") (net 2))
 (segment (start 100.5 114.3) (end 100.025489 114.774511) (width 0.25) (layer "F.Cu") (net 2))
 (segment (start 183.8 113.5) (end 184.8 113.5) (width 0.25) (layer "F.Cu") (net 2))
 (segment (start 53.34 124.46) (end 50.8 121.92) (width 0.25) (layer "F.Cu") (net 2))
 (segment (start 73.582139 127) (end 71.042139 124.46) (width 0.25) (layer "F.Cu") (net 2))
 (segment (start 182.88 112.58) (end 183.8 113.5) (width 0.25) (layer "F.Cu") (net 2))
 (segment (start 182.88 104.14) (end 190.5 104.14) (width 0.25) (layer "F.Cu") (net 2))
 (segment (start 99.06 116.84) (end 101.282142 114.617858) (width 0.25) (layer "B.Cu") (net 2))
 (segment (start 136.21 119.38) (end 99.06 119.38) (width 0.25) (layer "B.Cu") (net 2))
 (segment (start 100.964284 114.3) (end 99.06 114.3) (width 0.25) (layer "B.Cu") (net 2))
 (segment (start 99.06 119.38) (end 99.06 116.84) (width 0.25) (layer "B.Cu") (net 2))
 (segment (start 142.28 113.31) (end 136.21 119.38) (width 0.25) (layer "B.Cu") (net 2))
 (segment (start 101.282142 114.617858) (end 100.964284 114.3) (width 0.25) (layer "B.Cu") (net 2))
 (segment (start 102.184511 95.935489) (end 136.575489 95.935489) (width 0.25) (layer "F.Cu") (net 3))
 (segment (start 136.575489 95.935489) (end 145.43 104.79) (width 0.25) (layer "F.Cu") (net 3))
 (segment (start 91.44 111.76) (end 108.9 111.76) (width 0.25) (layer "F.Cu") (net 3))
 (segment (start 108.9 108.9) (end 104.14 104.14) (width 0.25) (layer "F.Cu") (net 3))
 (segment (start 93.98 104.14) (end 102.184511 95.935489) (width 0.25) (layer "F.Cu") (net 3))
 (segment (start 145.43 104.79) (end 145.43 109.81) (width 0.25) (layer "F.Cu") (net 3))
 (segment (start 83.82 104.14) (end 91.44 111.76) (width 0.25) (layer "F.Cu") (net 3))
 (segment (start 108.9 111.76) (end 108.9 108.9) (width 0.25) (layer "F.Cu") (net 3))
 (segment (start 51.64 104.14) (end 83.82 104.14) (width 0.25) (layer "F.Cu") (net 3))
 (segment (start 104.14 104.14) (end 93.98 104.14) (width 0.25) (layer "F.Cu") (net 3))
 (segment (start 104.66452 134.09548) (end 101.6 137.16) (width 0.25) (layer "F.Cu") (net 6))
 (segment (start 131.76 134.62) (end 131.23548 134.09548) (width 0.25) (layer "F.Cu") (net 6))
 (segment (start 101.28 136.84) (end 101.28 134.62) (width 0.25) (layer "F.Cu") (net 6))
 (segment (start 131.23548 134.09548) (end 104.66452 134.09548) (width 0.25) (layer "F.Cu") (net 6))
 (segment (start 101.6 137.16) (end 101.28 136.84) (width 0.25) (layer "F.Cu") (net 6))
 (segment (start 101.92 134.62) (end 101.92 119.570361) (width 0.25) (layer "F.Cu") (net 4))
 (segment (start 109.54 111.76) (end 109.54 99.36) (width 0.25) (layer "F.Cu") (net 4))
 (segment (start 101.92 134.429639) (end 101.92 134.62) (width 0.25) (layer "F.Cu") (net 4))
 (segment (start 109.54 99.36) (end 107.44 97.26) (width 0.25) (layer "F.Cu") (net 4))
 (segment (start 109.54 111.950361) (end 109.54 111.76) (width 0.25) (layer "F.Cu") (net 4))
 (segment (start 94.490361 127) (end 101.92 134.429639) (width 0.25) (layer "F.Cu") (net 4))
 (segment (start 101.92 119.570361) (end 109.54 111.950361) (width 0.25) (layer "F.Cu") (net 4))
 (segment (start 76.84 127) (end 94.490361 127) (width 0.25) (layer "F.Cu") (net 4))
 (segment (start 189.7 120) (end 189.7 121) (width 0.25) (layer "F.Cu") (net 1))
 (segment (start 188.78 121.92) (end 145.89 121.92) (width 0.25) (layer "F.Cu") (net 1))
 (segment (start 145.89 121.92) (end 142.28 118.31) (width 0.25) (layer "F.Cu") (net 1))
 (segment (start 189.7 121) (end 188.78 121.92) (width 0.25) (layer "F.Cu") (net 1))
 (segment (start 191.3 120) (end 191.3 118.325978) (width 0.25) (layer "F.Cu") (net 11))
 (segment (start 185.8 114.3) (end 190.5 109.6) (width 0.25) (layer "F.Cu") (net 11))
 (segment (start 184.8 114.3) (end 185.8 114.3) (width 0.25) (layer "F.Cu") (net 11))
 (segment (start 195.325978 114.3) (end 196.2 114.3) (width 0.25) (layer "F.Cu") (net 11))
 (segment (start 196.2 114.3) (end 195.2 114.3) (width 0.25) (layer "F.Cu") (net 11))
 (segment (start 191.3 118.325978) (end 195.325978 114.3) (width 0.25) (layer "F.Cu") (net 11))
 (segment (start 190.5 109.6) (end 190.5 108.6) (width 0.25) (layer "F.Cu") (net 11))
 (segment (start 195.2 114.3) (end 190.5 109.6) (width 0.25) (layer "F.Cu") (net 11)))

